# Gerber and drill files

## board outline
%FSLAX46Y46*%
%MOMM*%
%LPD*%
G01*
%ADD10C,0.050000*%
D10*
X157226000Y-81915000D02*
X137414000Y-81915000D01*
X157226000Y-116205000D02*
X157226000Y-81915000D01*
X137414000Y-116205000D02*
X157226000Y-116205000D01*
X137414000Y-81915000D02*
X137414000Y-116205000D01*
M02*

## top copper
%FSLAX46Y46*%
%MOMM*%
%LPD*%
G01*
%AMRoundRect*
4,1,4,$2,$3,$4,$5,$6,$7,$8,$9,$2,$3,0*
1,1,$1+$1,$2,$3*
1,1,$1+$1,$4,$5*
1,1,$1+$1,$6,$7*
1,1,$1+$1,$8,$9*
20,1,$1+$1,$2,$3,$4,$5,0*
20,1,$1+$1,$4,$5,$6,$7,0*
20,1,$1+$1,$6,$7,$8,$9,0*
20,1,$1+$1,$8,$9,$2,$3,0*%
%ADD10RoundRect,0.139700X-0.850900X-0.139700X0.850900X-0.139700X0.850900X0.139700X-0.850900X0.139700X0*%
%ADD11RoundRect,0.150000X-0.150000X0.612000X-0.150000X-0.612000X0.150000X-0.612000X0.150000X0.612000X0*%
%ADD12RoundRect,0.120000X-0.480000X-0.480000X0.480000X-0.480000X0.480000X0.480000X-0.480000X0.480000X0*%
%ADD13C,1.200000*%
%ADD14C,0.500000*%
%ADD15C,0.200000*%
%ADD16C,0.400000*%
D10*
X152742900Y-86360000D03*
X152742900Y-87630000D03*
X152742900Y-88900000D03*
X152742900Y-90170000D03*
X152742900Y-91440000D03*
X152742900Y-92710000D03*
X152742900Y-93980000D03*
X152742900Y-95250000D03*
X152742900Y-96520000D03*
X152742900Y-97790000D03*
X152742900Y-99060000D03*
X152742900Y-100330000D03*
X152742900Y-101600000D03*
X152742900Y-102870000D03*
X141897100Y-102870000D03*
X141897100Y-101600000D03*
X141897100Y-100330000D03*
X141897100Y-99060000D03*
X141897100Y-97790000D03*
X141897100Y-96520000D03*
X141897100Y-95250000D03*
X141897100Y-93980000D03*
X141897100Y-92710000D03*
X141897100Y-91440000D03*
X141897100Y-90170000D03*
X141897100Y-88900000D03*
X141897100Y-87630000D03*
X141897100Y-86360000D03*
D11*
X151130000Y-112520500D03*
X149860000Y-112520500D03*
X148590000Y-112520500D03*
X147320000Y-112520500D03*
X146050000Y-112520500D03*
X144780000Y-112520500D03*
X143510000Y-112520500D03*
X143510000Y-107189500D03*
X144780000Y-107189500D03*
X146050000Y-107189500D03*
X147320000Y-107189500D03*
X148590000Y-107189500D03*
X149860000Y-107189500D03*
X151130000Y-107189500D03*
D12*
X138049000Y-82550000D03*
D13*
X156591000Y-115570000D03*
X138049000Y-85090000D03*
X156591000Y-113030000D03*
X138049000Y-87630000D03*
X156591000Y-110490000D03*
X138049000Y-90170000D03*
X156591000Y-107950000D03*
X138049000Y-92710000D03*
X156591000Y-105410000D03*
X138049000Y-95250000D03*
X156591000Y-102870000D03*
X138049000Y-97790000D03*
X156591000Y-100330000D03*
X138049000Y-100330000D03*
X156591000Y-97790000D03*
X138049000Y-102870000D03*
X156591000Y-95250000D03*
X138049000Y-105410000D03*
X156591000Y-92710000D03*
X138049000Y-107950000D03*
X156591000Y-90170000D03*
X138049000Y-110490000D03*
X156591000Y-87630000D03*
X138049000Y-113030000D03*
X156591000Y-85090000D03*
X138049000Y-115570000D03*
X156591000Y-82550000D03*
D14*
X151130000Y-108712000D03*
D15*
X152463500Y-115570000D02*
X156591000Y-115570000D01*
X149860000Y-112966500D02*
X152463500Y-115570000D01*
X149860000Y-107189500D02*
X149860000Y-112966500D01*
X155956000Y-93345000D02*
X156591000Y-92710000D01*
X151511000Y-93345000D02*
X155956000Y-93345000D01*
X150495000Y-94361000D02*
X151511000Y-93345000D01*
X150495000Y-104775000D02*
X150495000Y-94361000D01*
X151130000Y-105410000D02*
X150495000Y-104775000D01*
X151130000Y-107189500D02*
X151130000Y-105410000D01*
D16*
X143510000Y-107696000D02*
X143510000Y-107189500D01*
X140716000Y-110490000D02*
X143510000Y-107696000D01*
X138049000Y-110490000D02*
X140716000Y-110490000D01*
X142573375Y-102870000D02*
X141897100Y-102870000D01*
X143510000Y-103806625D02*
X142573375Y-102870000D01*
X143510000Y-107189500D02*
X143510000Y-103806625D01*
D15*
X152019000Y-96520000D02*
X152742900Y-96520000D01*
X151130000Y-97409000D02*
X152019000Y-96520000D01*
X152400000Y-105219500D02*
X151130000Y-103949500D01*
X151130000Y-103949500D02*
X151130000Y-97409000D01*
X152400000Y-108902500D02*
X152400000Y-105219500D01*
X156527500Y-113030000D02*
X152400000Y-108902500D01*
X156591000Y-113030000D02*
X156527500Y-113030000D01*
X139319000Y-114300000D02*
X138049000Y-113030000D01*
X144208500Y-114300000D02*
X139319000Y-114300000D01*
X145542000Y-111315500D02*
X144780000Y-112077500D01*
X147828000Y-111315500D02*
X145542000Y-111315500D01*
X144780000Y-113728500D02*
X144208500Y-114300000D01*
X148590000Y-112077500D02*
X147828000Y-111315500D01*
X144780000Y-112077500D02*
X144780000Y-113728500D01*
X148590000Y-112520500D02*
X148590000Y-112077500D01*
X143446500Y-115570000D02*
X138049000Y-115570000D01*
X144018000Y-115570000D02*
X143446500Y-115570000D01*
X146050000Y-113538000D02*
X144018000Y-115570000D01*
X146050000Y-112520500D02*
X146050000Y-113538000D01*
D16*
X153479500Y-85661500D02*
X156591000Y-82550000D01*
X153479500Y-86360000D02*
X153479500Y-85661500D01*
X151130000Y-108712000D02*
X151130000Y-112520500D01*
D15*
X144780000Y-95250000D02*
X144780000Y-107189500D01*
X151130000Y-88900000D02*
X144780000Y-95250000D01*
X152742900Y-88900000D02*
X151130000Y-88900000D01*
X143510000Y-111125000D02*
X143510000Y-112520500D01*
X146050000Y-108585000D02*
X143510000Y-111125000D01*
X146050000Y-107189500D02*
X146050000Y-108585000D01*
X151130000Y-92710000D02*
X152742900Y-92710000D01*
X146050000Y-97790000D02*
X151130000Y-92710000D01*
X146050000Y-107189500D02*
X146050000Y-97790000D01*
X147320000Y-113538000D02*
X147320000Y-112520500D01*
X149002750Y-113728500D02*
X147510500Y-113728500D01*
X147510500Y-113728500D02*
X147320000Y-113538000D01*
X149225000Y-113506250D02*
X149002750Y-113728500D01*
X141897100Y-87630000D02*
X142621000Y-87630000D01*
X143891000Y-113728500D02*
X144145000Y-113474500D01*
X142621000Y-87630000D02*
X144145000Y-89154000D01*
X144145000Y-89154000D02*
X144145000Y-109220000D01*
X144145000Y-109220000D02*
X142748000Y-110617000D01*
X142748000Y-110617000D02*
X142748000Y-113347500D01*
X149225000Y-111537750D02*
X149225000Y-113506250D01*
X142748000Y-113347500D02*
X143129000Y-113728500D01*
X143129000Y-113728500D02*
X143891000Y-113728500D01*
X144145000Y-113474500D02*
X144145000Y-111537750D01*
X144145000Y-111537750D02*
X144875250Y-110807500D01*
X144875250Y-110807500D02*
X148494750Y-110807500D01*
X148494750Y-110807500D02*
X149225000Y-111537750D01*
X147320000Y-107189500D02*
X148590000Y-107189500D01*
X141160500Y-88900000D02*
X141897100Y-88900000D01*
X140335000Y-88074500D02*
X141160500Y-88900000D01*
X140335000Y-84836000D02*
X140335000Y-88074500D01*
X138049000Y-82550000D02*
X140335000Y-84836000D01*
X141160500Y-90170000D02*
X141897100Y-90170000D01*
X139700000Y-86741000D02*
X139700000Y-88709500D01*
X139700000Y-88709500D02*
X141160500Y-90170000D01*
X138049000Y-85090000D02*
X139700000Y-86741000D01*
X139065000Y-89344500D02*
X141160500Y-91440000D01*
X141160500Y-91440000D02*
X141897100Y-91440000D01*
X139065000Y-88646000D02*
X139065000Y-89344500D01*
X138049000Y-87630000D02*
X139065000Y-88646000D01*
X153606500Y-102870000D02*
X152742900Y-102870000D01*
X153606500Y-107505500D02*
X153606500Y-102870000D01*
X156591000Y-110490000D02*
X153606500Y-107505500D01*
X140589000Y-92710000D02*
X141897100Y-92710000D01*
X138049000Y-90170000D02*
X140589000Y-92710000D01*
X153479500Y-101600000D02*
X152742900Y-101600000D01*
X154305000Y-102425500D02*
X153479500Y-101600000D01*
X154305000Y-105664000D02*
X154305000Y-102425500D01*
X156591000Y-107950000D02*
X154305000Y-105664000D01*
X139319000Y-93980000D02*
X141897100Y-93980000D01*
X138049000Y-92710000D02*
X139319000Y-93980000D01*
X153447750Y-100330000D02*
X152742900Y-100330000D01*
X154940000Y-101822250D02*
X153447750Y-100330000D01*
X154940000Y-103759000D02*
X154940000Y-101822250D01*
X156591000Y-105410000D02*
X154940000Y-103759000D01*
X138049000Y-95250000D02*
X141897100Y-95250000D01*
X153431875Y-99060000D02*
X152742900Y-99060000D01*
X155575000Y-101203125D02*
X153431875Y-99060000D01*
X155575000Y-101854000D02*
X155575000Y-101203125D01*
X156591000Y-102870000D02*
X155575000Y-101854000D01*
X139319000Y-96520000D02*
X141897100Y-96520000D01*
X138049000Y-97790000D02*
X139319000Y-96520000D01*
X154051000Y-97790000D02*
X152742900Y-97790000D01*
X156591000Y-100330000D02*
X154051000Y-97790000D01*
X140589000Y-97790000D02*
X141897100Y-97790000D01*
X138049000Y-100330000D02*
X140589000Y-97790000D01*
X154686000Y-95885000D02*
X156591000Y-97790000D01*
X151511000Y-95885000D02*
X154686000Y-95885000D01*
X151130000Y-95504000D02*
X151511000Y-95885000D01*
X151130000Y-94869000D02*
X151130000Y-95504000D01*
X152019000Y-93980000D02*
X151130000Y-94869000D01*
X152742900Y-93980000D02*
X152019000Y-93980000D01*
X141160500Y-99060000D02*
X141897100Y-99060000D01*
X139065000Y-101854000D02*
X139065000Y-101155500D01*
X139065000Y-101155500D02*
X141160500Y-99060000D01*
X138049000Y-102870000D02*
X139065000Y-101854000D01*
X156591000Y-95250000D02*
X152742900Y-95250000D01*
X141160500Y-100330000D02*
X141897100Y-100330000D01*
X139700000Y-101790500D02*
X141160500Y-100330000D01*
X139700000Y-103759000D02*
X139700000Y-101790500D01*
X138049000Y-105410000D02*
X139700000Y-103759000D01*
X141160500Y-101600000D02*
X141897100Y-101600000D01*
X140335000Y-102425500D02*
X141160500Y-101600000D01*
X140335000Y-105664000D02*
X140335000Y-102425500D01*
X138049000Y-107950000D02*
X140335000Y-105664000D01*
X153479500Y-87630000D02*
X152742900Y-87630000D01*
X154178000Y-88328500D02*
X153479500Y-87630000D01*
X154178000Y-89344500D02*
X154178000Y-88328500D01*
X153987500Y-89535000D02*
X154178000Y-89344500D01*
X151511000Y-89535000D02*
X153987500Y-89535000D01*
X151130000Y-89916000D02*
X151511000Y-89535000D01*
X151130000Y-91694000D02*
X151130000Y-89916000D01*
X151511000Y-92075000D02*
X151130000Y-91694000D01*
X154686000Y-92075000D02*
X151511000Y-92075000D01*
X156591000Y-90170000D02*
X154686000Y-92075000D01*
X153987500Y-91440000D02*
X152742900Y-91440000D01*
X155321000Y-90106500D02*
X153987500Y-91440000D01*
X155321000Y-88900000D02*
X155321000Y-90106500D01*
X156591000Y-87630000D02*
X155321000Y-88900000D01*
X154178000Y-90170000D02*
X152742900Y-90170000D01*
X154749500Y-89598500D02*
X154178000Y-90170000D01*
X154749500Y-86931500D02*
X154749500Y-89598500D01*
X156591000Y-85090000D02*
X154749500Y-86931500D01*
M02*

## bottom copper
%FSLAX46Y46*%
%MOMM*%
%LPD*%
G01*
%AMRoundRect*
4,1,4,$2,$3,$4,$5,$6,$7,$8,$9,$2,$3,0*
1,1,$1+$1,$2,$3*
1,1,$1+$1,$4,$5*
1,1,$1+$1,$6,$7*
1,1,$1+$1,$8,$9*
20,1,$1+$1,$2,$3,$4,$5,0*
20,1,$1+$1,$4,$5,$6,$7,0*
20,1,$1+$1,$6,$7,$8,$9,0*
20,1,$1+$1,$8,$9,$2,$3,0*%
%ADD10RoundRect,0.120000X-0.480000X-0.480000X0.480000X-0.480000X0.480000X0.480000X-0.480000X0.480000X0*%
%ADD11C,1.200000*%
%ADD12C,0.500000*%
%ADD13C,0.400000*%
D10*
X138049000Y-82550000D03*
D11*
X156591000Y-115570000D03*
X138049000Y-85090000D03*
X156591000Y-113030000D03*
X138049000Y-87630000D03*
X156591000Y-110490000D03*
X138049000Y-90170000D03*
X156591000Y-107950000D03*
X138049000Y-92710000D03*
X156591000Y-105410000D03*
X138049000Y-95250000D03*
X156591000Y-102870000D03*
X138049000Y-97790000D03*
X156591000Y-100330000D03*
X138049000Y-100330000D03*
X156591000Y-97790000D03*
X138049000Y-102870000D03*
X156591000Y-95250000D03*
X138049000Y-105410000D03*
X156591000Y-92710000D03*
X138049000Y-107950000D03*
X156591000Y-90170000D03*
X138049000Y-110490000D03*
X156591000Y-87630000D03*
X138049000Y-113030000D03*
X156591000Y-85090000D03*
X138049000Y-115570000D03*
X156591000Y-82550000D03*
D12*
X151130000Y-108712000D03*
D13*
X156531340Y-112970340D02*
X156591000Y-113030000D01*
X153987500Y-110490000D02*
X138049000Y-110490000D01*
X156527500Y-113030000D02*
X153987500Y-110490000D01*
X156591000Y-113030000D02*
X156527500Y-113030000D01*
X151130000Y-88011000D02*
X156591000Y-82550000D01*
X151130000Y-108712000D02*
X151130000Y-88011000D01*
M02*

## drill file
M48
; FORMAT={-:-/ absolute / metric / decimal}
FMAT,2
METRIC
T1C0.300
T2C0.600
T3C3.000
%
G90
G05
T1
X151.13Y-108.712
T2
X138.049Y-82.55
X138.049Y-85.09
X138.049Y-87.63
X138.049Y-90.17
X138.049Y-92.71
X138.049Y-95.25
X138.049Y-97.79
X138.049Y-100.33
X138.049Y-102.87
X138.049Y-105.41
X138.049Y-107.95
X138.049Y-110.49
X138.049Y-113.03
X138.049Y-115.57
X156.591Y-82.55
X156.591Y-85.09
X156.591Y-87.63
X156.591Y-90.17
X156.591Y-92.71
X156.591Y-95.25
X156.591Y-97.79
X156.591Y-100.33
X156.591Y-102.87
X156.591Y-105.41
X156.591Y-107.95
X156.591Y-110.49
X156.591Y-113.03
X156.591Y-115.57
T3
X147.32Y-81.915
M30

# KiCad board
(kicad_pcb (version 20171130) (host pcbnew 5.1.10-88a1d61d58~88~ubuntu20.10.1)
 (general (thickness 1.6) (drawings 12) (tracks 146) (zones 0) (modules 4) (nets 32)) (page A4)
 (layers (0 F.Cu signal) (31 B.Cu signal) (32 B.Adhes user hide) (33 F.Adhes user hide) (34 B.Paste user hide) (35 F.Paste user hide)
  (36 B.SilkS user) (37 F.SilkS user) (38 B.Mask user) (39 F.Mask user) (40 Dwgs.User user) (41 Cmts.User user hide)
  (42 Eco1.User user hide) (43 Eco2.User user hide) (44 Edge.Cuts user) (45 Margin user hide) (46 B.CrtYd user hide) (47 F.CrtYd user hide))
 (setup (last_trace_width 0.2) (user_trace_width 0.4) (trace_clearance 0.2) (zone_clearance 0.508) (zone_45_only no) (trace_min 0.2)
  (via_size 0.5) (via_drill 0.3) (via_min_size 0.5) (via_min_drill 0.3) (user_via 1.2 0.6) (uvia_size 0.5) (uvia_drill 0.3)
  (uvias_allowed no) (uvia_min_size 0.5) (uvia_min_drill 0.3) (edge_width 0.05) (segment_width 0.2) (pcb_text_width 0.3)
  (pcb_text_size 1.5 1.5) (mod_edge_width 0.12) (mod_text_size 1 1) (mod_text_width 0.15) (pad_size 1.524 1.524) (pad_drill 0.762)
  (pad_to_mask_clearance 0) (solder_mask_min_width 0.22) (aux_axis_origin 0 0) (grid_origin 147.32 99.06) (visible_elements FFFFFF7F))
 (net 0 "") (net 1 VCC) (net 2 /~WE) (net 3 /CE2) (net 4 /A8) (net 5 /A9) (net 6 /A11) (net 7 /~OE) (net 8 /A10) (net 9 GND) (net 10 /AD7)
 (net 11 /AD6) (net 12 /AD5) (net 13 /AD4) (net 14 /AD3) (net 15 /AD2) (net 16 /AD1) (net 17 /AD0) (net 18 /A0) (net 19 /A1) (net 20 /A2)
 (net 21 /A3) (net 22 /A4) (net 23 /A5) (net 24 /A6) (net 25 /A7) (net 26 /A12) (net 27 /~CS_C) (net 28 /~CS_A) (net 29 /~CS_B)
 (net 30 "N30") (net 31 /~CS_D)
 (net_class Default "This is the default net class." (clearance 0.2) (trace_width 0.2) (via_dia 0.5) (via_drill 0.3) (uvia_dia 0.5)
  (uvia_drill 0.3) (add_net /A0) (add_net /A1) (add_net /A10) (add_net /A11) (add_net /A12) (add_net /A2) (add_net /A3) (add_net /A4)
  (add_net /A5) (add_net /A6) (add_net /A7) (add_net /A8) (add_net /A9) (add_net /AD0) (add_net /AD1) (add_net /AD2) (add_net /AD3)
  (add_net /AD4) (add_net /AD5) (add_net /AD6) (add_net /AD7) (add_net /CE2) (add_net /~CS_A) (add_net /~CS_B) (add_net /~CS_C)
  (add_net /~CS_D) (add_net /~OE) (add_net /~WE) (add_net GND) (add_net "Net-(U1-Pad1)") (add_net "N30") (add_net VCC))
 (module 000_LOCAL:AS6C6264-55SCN (layer F.Cu) (at 147.32 94.615)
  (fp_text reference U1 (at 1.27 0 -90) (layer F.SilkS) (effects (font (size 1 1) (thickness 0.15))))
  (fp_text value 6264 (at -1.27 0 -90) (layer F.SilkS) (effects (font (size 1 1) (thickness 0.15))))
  (pad 28 smd roundrect (at 5.4229 -8.255) (size 1.9812 0.5588) (layers F.Cu F.Paste F.Mask) (roundrect_rratio 0.25) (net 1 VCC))
  (pad 27 smd roundrect (at 5.4229 -6.985) (size 1.9812 0.5588) (layers F.Cu F.Paste F.Mask) (roundrect_rratio 0.25) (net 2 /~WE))
  (pad 26 smd roundrect (at 5.4229 -5.715) (size 1.9812 0.5588) (layers F.Cu F.Paste F.Mask) (roundrect_rratio 0.25) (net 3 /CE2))
  (pad 25 smd roundrect (at 5.4229 -4.445) (size 1.9812 0.5588) (layers F.Cu F.Paste F.Mask) (roundrect_rratio 0.25) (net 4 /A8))
  (pad 24 smd roundrect (at 5.4229 -3.175) (size 1.9812 0.5588) (layers F.Cu F.Paste F.Mask) (roundrect_rratio 0.25) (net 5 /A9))
  (pad 23 smd roundrect (at 5.4229 -1.905) (size 1.9812 0.5588) (layers F.Cu F.Paste F.Mask) (roundrect_rratio 0.25) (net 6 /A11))
  (pad 22 smd roundrect (at 5.4229 -0.635) (size 1.9812 0.5588) (layers F.Cu F.Paste F.Mask) (roundrect_rratio 0.25) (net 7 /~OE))
  (pad 21 smd roundrect (at 5.4229 0.635) (size 1.9812 0.5588) (layers F.Cu F.Paste F.Mask) (roundrect_rratio 0.25) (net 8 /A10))
  (pad 20 smd roundrect (at 5.4229 1.905) (size 1.9812 0.5588) (layers F.Cu F.Paste F.Mask) (roundrect_rratio 0.25) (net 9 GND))
  (pad 19 smd roundrect (at 5.4229 3.175) (size 1.9812 0.5588) (layers F.Cu F.Paste F.Mask) (roundrect_rratio 0.25) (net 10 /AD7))
  (pad 18 smd roundrect (at 5.4229 4.445) (size 1.9812 0.5588) (layers F.Cu F.Paste F.Mask) (roundrect_rratio 0.25) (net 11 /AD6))
  (pad 17 smd roundrect (at 5.4229 5.715) (size 1.9812 0.5588) (layers F.Cu F.Paste F.Mask) (roundrect_rratio 0.25) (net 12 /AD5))
  (pad 16 smd roundrect (at 5.4229 6.985) (size 1.9812 0.5588) (layers F.Cu F.Paste F.Mask) (roundrect_rratio 0.25) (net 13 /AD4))
  (pad 15 smd roundrect (at 5.4229 8.255) (size 1.9812 0.5588) (layers F.Cu F.Paste F.Mask) (roundrect_rratio 0.25) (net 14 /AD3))
  (pad 14 smd roundrect (at -5.4229 8.255) (size 1.9812 0.5588) (layers F.Cu F.Paste F.Mask) (roundrect_rratio 0.25) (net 9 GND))
  (pad 13 smd roundrect (at -5.4229 6.985) (size 1.9812 0.5588) (layers F.Cu F.Paste F.Mask) (roundrect_rratio 0.25) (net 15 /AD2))
  (pad 12 smd roundrect (at -5.4229 5.715) (size 1.9812 0.5588) (layers F.Cu F.Paste F.Mask) (roundrect_rratio 0.25) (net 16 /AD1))
  (pad 11 smd roundrect (at -5.4229 4.445) (size 1.9812 0.5588) (layers F.Cu F.Paste F.Mask) (roundrect_rratio 0.25) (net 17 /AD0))
  (pad 10 smd roundrect (at -5.4229 3.175) (size 1.9812 0.5588) (layers F.Cu F.Paste F.Mask) (roundrect_rratio 0.25) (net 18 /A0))
  (pad 9 smd roundrect (at -5.4229 1.905) (size 1.9812 0.5588) (layers F.Cu F.Paste F.Mask) (roundrect_rratio 0.25) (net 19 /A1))
  (pad 8 smd roundrect (at -5.4229 0.635) (size 1.9812 0.5588) (layers F.Cu F.Paste F.Mask) (roundrect_rratio 0.25) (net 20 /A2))
  (pad 7 smd roundrect (at -5.4229 -0.635) (size 1.9812 0.5588) (layers F.Cu F.Paste F.Mask) (roundrect_rratio 0.25) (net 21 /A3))
  (pad 6 smd roundrect (at -5.4229 -1.905) (size 1.9812 0.5588) (layers F.Cu F.Paste F.Mask) (roundrect_rratio 0.25) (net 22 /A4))
  (pad 5 smd roundrect (at -5.4229 -3.175) (size 1.9812 0.5588) (layers F.Cu F.Paste F.Mask) (roundrect_rratio 0.25) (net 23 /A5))
  (pad 4 smd roundrect (at -5.4229 -4.445) (size 1.9812 0.5588) (layers F.Cu F.Paste F.Mask) (roundrect_rratio 0.25) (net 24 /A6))
  (pad 3 smd roundrect (at -5.4229 -5.715) (size 1.9812 0.5588) (layers F.Cu F.Paste F.Mask) (roundrect_rratio 0.25) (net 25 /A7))
  (pad 2 smd roundrect (at -5.4229 -6.985) (size 1.9812 0.5588) (layers F.Cu F.Paste F.Mask) (roundrect_rratio 0.25) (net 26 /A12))
  (pad 1 smd roundrect (at -5.4229 -8.255) (size 1.9812 0.5588) (layers F.Cu F.Paste F.Mask) (roundrect_rratio 0.25)))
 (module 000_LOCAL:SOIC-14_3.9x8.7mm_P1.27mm (layer F.Cu) (at 147.32 109.855 270) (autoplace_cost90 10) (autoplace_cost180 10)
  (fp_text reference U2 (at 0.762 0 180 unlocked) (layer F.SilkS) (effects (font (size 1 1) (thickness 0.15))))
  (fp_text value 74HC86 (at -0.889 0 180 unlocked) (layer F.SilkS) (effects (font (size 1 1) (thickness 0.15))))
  (pad 14 smd roundrect (at 2.6655 -3.81 270) (size 1.524 0.6) (layers F.Cu F.Paste F.Mask) (roundrect_rratio 0.25) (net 1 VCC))
  (pad 13 smd roundrect (at 2.6655 -2.54 270) (size 1.524 0.6) (layers F.Cu F.Paste F.Mask) (roundrect_rratio 0.25) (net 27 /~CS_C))
  (pad 12 smd roundrect (at 2.6655 -1.27 270) (size 1.524 0.6) (layers F.Cu F.Paste F.Mask) (roundrect_rratio 0.25) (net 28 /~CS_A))
  (pad 11 smd roundrect (at 2.6655 0 270) (size 1.524 0.6) (layers F.Cu F.Paste F.Mask) (roundrect_rratio 0.25) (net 26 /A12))
  (pad 10 smd roundrect (at 2.6655 1.27 270) (size 1.524 0.6) (layers F.Cu F.Paste F.Mask) (roundrect_rratio 0.25) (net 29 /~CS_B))
  (pad 9 smd roundrect (at 2.6655 2.54 270) (size 1.524 0.6) (layers F.Cu F.Paste F.Mask) (roundrect_rratio 0.25) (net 28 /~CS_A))
  (pad 8 smd roundrect (at 2.6655 3.81 270) (size 1.524 0.6) (layers F.Cu F.Paste F.Mask) (roundrect_rratio 0.25) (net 6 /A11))
  (pad 7 smd roundrect (at -2.6655 3.81 270) (size 1.524 0.6) (layers F.Cu F.Paste F.Mask) (roundrect_rratio 0.25) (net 9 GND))
  (pad 6 smd roundrect (at -2.6655 2.54 270) (size 1.524 0.6) (layers F.Cu F.Paste F.Mask) (roundrect_rratio 0.25) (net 3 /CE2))
  (pad 5 smd roundrect (at -2.6655 1.27 270) (size 1.524 0.6) (layers F.Cu F.Paste F.Mask) (roundrect_rratio 0.25) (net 6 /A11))
  (pad 4 smd roundrect (at -2.6655 0 270) (size 1.524 0.6) (layers F.Cu F.Paste F.Mask) (roundrect_rratio 0.25) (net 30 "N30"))
  (pad 3 smd roundrect (at -2.6655 -1.27 270) (size 1.524 0.6) (layers F.Cu F.Paste F.Mask) (roundrect_rratio 0.25) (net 30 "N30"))
  (pad 2 smd roundrect (at -2.6655 -2.54 270) (size 1.524 0.6) (layers F.Cu F.Paste F.Mask) (roundrect_rratio 0.25) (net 27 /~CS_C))
  (pad 1 smd roundrect (at -2.6655 -3.81 270) (size 1.524 0.6) (layers F.Cu F.Paste F.Mask) (roundrect_rratio 0.25) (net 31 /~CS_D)))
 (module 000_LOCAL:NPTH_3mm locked (layer F.Cu) (at 147.32 81.915)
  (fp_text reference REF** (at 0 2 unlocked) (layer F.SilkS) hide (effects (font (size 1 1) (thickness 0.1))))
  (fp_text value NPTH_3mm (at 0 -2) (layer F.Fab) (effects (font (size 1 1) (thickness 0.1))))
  (pad "" np_thru_hole circle (at 0 0) (size 3 3) (drill 3) (layers *.Cu *.Mask)))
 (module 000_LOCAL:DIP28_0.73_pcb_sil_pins (layer F.Cu) (at 147.32 99.06)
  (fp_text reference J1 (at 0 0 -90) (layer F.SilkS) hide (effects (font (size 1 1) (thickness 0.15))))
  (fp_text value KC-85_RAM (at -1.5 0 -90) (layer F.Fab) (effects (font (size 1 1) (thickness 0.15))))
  (pad 1 thru_hole roundrect (at -9.271 -16.51) (size 1.2 1.2) (drill 0.6) (layers *.Cu *.Mask) (roundrect_rratio 0.1) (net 25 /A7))
  (pad 15 thru_hole circle (at 9.271 16.51) (size 1.2 1.2) (drill 0.6) (layers *.Cu *.Mask) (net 27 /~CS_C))
  (pad 2 thru_hole circle (at -9.271 -13.97) (size 1.2 1.2) (drill 0.6) (layers *.Cu *.Mask) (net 24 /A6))
  (pad 16 thru_hole circle (at 9.271 13.97) (size 1.2 1.2) (drill 0.6) (layers *.Cu *.Mask) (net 9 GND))
  (pad 3 thru_hole circle (at -9.271 -11.43) (size 1.2 1.2) (drill 0.6) (layers *.Cu *.Mask) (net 23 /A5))
  (pad 17 thru_hole circle (at 9.271 11.43) (size 1.2 1.2) (drill 0.6) (layers *.Cu *.Mask) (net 14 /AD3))
  (pad 4 thru_hole circle (at -9.271 -8.89) (size 1.2 1.2) (drill 0.6) (layers *.Cu *.Mask) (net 22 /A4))
  (pad 18 thru_hole circle (at 9.271 8.89) (size 1.2 1.2) (drill 0.6) (layers *.Cu *.Mask) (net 13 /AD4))
  (pad 5 thru_hole circle (at -9.271 -6.35) (size 1.2 1.2) (drill 0.6) (layers *.Cu *.Mask) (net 21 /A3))
  (pad 19 thru_hole circle (at 9.271 6.35) (size 1.2 1.2) (drill 0.6) (layers *.Cu *.Mask) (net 12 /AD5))
  (pad 6 thru_hole circle (at -9.271 -3.81) (size 1.2 1.2) (drill 0.6) (layers *.Cu *.Mask) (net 20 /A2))
  (pad 20 thru_hole circle (at 9.271 3.81) (size 1.2 1.2) (drill 0.6) (layers *.Cu *.Mask) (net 11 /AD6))
  (pad 7 thru_hole circle (at -9.271 -1.27) (size 1.2 1.2) (drill 0.6) (layers *.Cu *.Mask) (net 19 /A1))
  (pad 21 thru_hole circle (at 9.271 1.27) (size 1.2 1.2) (drill 0.6) (layers *.Cu *.Mask) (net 10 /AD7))
  (pad 8 thru_hole circle (at -9.271 1.27) (size 1.2 1.2) (drill 0.6) (layers *.Cu *.Mask) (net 18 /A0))
  (pad 22 thru_hole circle (at 9.271 -1.27) (size 1.2 1.2) (drill 0.6) (layers *.Cu *.Mask) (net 7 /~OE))
  (pad 9 thru_hole circle (at -9.271 3.81) (size 1.2 1.2) (drill 0.6) (layers *.Cu *.Mask) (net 17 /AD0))
  (pad 23 thru_hole circle (at 9.271 -3.81) (size 1.2 1.2) (drill 0.6) (layers *.Cu *.Mask) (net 8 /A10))
  (pad 10 thru_hole circle (at -9.271 6.35) (size 1.2 1.2) (drill 0.6) (layers *.Cu *.Mask) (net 16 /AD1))
  (pad 24 thru_hole circle (at 9.271 -6.35) (size 1.2 1.2) (drill 0.6) (layers *.Cu *.Mask) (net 31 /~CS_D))
  (pad 11 thru_hole circle (at -9.271 8.89) (size 1.2 1.2) (drill 0.6) (layers *.Cu *.Mask) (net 15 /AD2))
  (pad 25 thru_hole circle (at 9.271 -8.89) (size 1.2 1.2) (drill 0.6) (layers *.Cu *.Mask) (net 2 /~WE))
  (pad 12 thru_hole circle (at -9.271 11.43) (size 1.2 1.2) (drill 0.6) (layers *.Cu *.Mask) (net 9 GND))
  (pad 26 thru_hole circle (at 9.271 -11.43) (size 1.2 1.2) (drill 0.6) (layers *.Cu *.Mask) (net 5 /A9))
  (pad 13 thru_hole circle (at -9.271 13.97) (size 1.2 1.2) (drill 0.6) (layers *.Cu *.Mask) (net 28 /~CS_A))
  (pad 27 thru_hole circle (at 9.271 -13.97) (size 1.2 1.2) (drill 0.6) (layers *.Cu *.Mask) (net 4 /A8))
  (pad 14 thru_hole circle (at -9.271 16.51) (size 1.2 1.2) (drill 0.6) (layers *.Cu *.Mask) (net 29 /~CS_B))
  (pad 28 thru_hole circle (at 9.271 -16.51) (size 1.2 1.2) (drill 0.6) (layers *.Cu *.Mask) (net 1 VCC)))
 (gr_line (start 157.226 81.915) (end 137.414 81.915) (layer Edge.Cuts) (width 0.05))
 (gr_line (start 157.226 116.205) (end 157.226 81.915) (layer Edge.Cuts) (width 0.05))
 (gr_line (start 137.414 116.205) (end 157.226 116.205) (layer Edge.Cuts) (width 0.05))
 (gr_line (start 137.414 81.915) (end 137.414 116.205) (layer Edge.Cuts) (width 0.05))
 (segment (start 152.4635 115.57) (end 156.591 115.57) (width 0.2) (layer F.Cu) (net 27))
 (segment (start 149.86 112.9665) (end 152.4635 115.57) (width 0.2) (layer F.Cu) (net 27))
 (segment (start 149.86 107.1895) (end 149.86 112.9665) (width 0.2) (layer F.Cu) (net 27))
 (segment (start 155.956 93.345) (end 156.591 92.71) (width 0.2) (layer F.Cu) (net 31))
 (segment (start 151.511 93.345) (end 155.956 93.345) (width 0.2) (layer F.Cu) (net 31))
 (segment (start 150.495 94.361) (end 151.511 93.345) (width 0.2) (layer F.Cu) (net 31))
 (segment (start 150.495 104.775) (end 150.495 94.361) (width 0.2) (layer F.Cu) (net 31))
 (segment (start 151.13 105.41) (end 150.495 104.775) (width 0.2) (layer F.Cu) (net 31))
 (segment (start 151.13 107.1895) (end 151.13 105.41) (width 0.2) (layer F.Cu) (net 31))
 (segment (start 156.53134 112.97034) (end 156.591 113.03) (width 0.4) (layer B.Cu) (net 9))
 (segment (start 143.51 107.696) (end 143.51 107.1895) (width 0.4) (layer F.Cu) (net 9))
 (segment (start 140.716 110.49) (end 143.51 107.696) (width 0.4) (layer F.Cu) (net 9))
 (segment (start 138.049 110.49) (end 140.716 110.49) (width 0.4) (layer F.Cu) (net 9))
 (segment (start 142.573375 102.87) (end 141.8971 102.87) (width 0.4) (layer F.Cu) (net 9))
 (segment (start 143.51 103.806625) (end 142.573375 102.87) (width 0.4) (layer F.Cu) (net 9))
 (segment (start 143.51 107.1895) (end 143.51 103.806625) (width 0.4) (layer F.Cu) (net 9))
 (segment (start 152.019 96.52) (end 152.7429 96.52) (width 0.2) (layer F.Cu) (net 9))
 (segment (start 151.13 97.409) (end 152.019 96.52) (width 0.2) (layer F.Cu) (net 9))
 (segment (start 152.4 105.2195) (end 151.13 103.9495) (width 0.2) (layer F.Cu) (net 9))
 (segment (start 151.13 103.9495) (end 151.13 97.409) (width 0.2) (layer F.Cu) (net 9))
 (segment (start 152.4 108.9025) (end 152.4 105.2195) (width 0.2) (layer F.Cu) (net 9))
 (segment (start 156.5275 113.03) (end 152.4 108.9025) (width 0.2) (layer F.Cu) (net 9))
 (segment (start 156.591 113.03) (end 156.5275 113.03) (width 0.2) (layer F.Cu) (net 9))
 (segment (start 153.9875 110.49) (end 138.049 110.49) (width 0.4) (layer B.Cu) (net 9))
 (segment (start 156.5275 113.03) (end 153.9875 110.49) (width 0.4) (layer B.Cu) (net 9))
 (segment (start 156.591 113.03) (end 156.5275 113.03) (width 0.4) (layer B.Cu) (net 9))
 (segment (start 139.319 114.3) (end 138.049 113.03) (width 0.2) (layer F.Cu) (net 28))
 (segment (start 144.2085 114.3) (end 139.319 114.3) (width 0.2) (layer F.Cu) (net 28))
 (segment (start 145.542 111.3155) (end 144.78 112.0775) (width 0.2) (layer F.Cu) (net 28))
 (segment (start 147.828 111.3155) (end 145.542 111.3155) (width 0.2) (layer F.Cu) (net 28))
 (segment (start 144.78 113.7285) (end 144.2085 114.3) (width 0.2) (layer F.Cu) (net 28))
 (segment (start 148.59 112.0775) (end 147.828 111.3155) (width 0.2) (layer F.Cu) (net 28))
 (segment (start 144.78 112.0775) (end 144.78 113.7285) (width 0.2) (layer F.Cu) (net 28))
 (segment (start 148.59 112.5205) (end 148.59 112.0775) (width 0.2) (layer F.Cu) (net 28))
 (segment (start 143.4465 115.57) (end 138.049 115.57) (width 0.2) (layer F.Cu) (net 29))
 (segment (start 144.018 115.57) (end 143.4465 115.57) (width 0.2) (layer F.Cu) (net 29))
 (segment (start 146.05 113.538) (end 144.018 115.57) (width 0.2) (layer F.Cu) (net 29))
 (segment (start 146.05 112.5205) (end 146.05 113.538) (width 0.2) (layer F.Cu) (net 29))
 (segment (start 153.4795 85.6615) (end 156.591 82.55) (width 0.4) (layer F.Cu) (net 1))
 (segment (start 153.4795 86.36) (end 153.4795 85.6615) (width 0.4) (layer F.Cu) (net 1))
 (segment (start 151.13 88.011) (end 156.591 82.55) (width 0.4) (layer B.Cu) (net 1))
 (segment (start 151.13 108.712) (end 151.13 88.011) (width 0.4) (layer B.Cu) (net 1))
 (segment (start 151.13 108.712) (end 151.13 112.5205) (width 0.4) (layer F.Cu) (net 1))
 (via (at 151.13 108.712) (size 0.5) (drill 0.3) (layers F.Cu B.Cu) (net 1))
 (segment (start 144.78 95.25) (end 144.78 107.1895) (width 0.2) (layer F.Cu) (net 3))
 (segment (start 151.13 88.9) (end 144.78 95.25) (width 0.2) (layer F.Cu) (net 3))
 (segment (start 152.7429 88.9) (end 151.13 88.9) (width 0.2) (layer F.Cu) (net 3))
 (segment (start 143.51 111.125) (end 143.51 112.5205) (width 0.2) (layer F.Cu) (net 6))
 (segment (start 146.05 108.585) (end 143.51 111.125) (width 0.2) (layer F.Cu) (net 6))
 (segment (start 146.05 107.1895) (end 146.05 108.585) (width 0.2) (layer F.Cu) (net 6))
 (segment (start 151.13 92.71) (end 152.7429 92.71) (width 0.2) (layer F.Cu) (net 6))
 (segment (start 146.05 97.79) (end 151.13 92.71) (width 0.2) (layer F.Cu) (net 6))
 (segment (start 146.05 107.1895) (end 146.05 97.79) (width 0.2) (layer F.Cu) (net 6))
 (segment (start 147.32 113.538) (end 147.32 112.5205) (width 0.2) (layer F.Cu) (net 26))
 (segment (start 149.00275 113.7285) (end 147.5105 113.7285) (width 0.2) (layer F.Cu) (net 26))
 (segment (start 147.5105 113.7285) (end 147.32 113.538) (width 0.2) (layer F.Cu) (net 26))
 (segment (start 149.225 113.50625) (end 149.00275 113.7285) (width 0.2) (layer F.Cu) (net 26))
 (segment (start 141.8971 87.63) (end 142.621 87.63) (width 0.2) (layer F.Cu) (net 26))
 (segment (start 143.891 113.7285) (end 144.145 113.4745) (width 0.2) (layer F.Cu) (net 26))
 (segment (start 142.621 87.63) (end 144.145 89.154) (width 0.2) (layer F.Cu) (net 26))
 (segment (start 144.145 89.154) (end 144.145 109.22) (width 0.2) (layer F.Cu) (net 26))
 (segment (start 144.145 109.22) (end 142.748 110.617) (width 0.2) (layer F.Cu) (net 26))
 (segment (start 142.748 110.617) (end 142.748 113.3475) (width 0.2) (layer F.Cu) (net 26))
 (segment (start 149.225 111.53775) (end 149.225 113.50625) (width 0.2) (layer F.Cu) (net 26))
 (segment (start 142.748 113.3475) (end 143.129 113.7285) (width 0.2) (layer F.Cu) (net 26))
 (segment (start 143.129 113.7285) (end 143.891 113.7285) (width 0.2) (layer F.Cu) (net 26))
 (segment (start 144.145 113.4745) (end 144.145 111.53775) (width 0.2) (layer F.Cu) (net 26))
 (segment (start 144.145 111.53775) (end 144.87525 110.8075) (width 0.2) (layer F.Cu) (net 26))
 (segment (start 144.87525 110.8075) (end 148.49475 110.8075) (width 0.2) (layer F.Cu) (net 26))
 (segment (start 148.49475 110.8075) (end 149.225 111.53775) (width 0.2) (layer F.Cu) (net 26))
 (segment (start 147.32 107.1895) (end 148.59 107.1895) (width 0.2) (layer F.Cu) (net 30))
 (segment (start 141.1605 88.9) (end 141.8971 88.9) (width 0.2) (layer F.Cu) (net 25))
 (segment (start 140.335 88.0745) (end 141.1605 88.9) (width 0.2) (layer F.Cu) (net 25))
 (segment (start 140.335 84.836) (end 140.335 88.0745) (width 0.2) (layer F.Cu) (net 25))
 (segment (start 138.049 82.55) (end 140.335 84.836) (width 0.2) (layer F.Cu) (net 25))
 (segment (start 141.1605 90.17) (end 141.8971 90.17) (width 0.2) (layer F.Cu) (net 24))
 (segment (start 139.7 86.741) (end 139.7 88.7095) (width 0.2) (layer F.Cu) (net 24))
 (segment (start 139.7 88.7095) (end 141.1605 90.17) (width 0.2) (layer F.Cu) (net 24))
 (segment (start 138.049 85.09) (end 139.7 86.741) (width 0.2) (layer F.Cu) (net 24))
 (segment (start 139.065 89.3445) (end 141.1605 91.44) (width 0.2) (layer F.Cu) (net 23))
 (segment (start 141.1605 91.44) (end 141.8971 91.44) (width 0.2) (layer F.Cu) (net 23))
 (segment (start 139.065 88.646) (end 139.065 89.3445) (width 0.2) (layer F.Cu) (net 23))
 (segment (start 138.049 87.63) (end 139.065 88.646) (width 0.2) (layer F.Cu) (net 23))
 (segment (start 153.6065 102.87) (end 152.7429 102.87) (width 0.2) (layer F.Cu) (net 14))
 (segment (start 153.6065 107.5055) (end 153.6065 102.87) (width 0.2) (layer F.Cu) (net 14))
 (segment (start 156.591 110.49) (end 153.6065 107.5055) (width 0.2) (layer F.Cu) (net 14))
 (segment (start 140.589 92.71) (end 141.8971 92.71) (width 0.2) (layer F.Cu) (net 22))
 (segment (start 138.049 90.17) (end 140.589 92.71) (width 0.2) (layer F.Cu) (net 22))
 (segment (start 153.4795 101.6) (end 152.7429 101.6) (width 0.2) (layer F.Cu) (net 13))
 (segment (start 154.305 102.4255) (end 153.4795 101.6) (width 0.2) (layer F.Cu) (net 13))
 (segment (start 154.305 105.664) (end 154.305 102.4255) (width 0.2) (layer F.Cu) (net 13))
 (segment (start 156.591 107.95) (end 154.305 105.664) (width 0.2) (layer F.Cu) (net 13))
 (segment (start 139.319 93.98) (end 141.8971 93.98) (width 0.2) (layer F.Cu) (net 21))
 (segment (start 138.049 92.71) (end 139.319 93.98) (width 0.2) (layer F.Cu) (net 21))
 (segment (start 153.44775 100.33) (end 152.7429 100.33) (width 0.2) (layer F.Cu) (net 12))
 (segment (start 154.94 101.82225) (end 153.44775 100.33) (width 0.2) (layer F.Cu) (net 12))
 (segment (start 154.94 103.759) (end 154.94 101.82225) (width 0.2) (layer F.Cu) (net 12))
 (segment (start 156.591 105.41) (end 154.94 103.759) (width 0.2) (layer F.Cu) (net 12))
 (segment (start 138.049 95.25) (end 141.8971 95.25) (width 0.2) (layer F.Cu) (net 20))
 (segment (start 153.431875 99.06) (end 152.7429 99.06) (width 0.2) (layer F.Cu) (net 11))
 (segment (start 155.575 101.203125) (end 153.431875 99.06) (width 0.2) (layer F.Cu) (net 11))
 (segment (start 155.575 101.854) (end 155.575 101.203125) (width 0.2) (layer F.Cu) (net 11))
 (segment (start 156.591 102.87) (end 155.575 101.854) (width 0.2) (layer F.Cu) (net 11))
 (segment (start 139.319 96.52) (end 141.8971 96.52) (width 0.2) (layer F.Cu) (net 19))
 (segment (start 138.049 97.79) (end 139.319 96.52) (width 0.2) (layer F.Cu) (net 19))
 (segment (start 154.051 97.79) (end 152.7429 97.79) (width 0.2) (layer F.Cu) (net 10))
 (segment (start 156.591 100.33) (end 154.051 97.79) (width 0.2) (layer F.Cu) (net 10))
 (segment (start 140.589 97.79) (end 141.8971 97.79) (width 0.2) (layer F.Cu) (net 18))
 (segment (start 138.049 100.33) (end 140.589 97.79) (width 0.2) (layer F.Cu) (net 18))
 (segment (start 154.686 95.885) (end 156.591 97.79) (width 0.2) (layer F.Cu) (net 7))
 (segment (start 151.511 95.885) (end 154.686 95.885) (width 0.2) (layer F.Cu) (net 7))
 (segment (start 151.13 95.504) (end 151.511 95.885) (width 0.2) (layer F.Cu) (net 7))
 (segment (start 151.13 94.869) (end 151.13 95.504) (width 0.2) (layer F.Cu) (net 7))
 (segment (start 152.019 93.98) (end 151.13 94.869) (width 0.2) (layer F.Cu) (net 7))
 (segment (start 152.7429 93.98) (end 152.019 93.98) (width 0.2) (layer F.Cu) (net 7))
 (segment (start 141.1605 99.06) (end 141.8971 99.06) (width 0.2) (layer F.Cu) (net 17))
 (segment (start 139.065 101.854) (end 139.065 101.1555) (width 0.2) (layer F.Cu) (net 17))
 (segment (start 139.065 101.1555) (end 141.1605 99.06) (width 0.2) (layer F.Cu) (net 17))
 (segment (start 138.049 102.87) (end 139.065 101.854) (width 0.2) (layer F.Cu) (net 17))
 (segment (start 156.591 95.25) (end 152.7429 95.25) (width 0.2) (layer F.Cu) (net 8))
 (segment (start 141.1605 100.33) (end 141.8971 100.33) (width 0.2) (layer F.Cu) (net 16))
 (segment (start 139.7 101.7905) (end 141.1605 100.33) (width 0.2) (layer F.Cu) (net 16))
 (segment (start 139.7 103.759) (end 139.7 101.7905) (width 0.2) (layer F.Cu) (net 16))
 (segment (start 138.049 105.41) (end 139.7 103.759) (width 0.2) (layer F.Cu) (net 16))
 (segment (start 141.1605 101.6) (end 141.8971 101.6) (width 0.2) (layer F.Cu) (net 15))
 (segment (start 140.335 102.4255) (end 141.1605 101.6) (width 0.2) (layer F.Cu) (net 15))
 (segment (start 140.335 105.664) (end 140.335 102.4255) (width 0.2) (layer F.Cu) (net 15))
 (segment (start 138.049 107.95) (end 140.335 105.664) (width 0.2) (layer F.Cu) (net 15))
 (segment (start 153.4795 87.63) (end 152.7429 87.63) (width 0.2) (layer F.Cu) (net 2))
 (segment (start 154.178 88.3285) (end 153.4795 87.63) (width 0.2) (layer F.Cu) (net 2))
 (segment (start 154.178 89.3445) (end 154.178 88.3285) (width 0.2) (layer F.Cu) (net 2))
 (segment (start 153.9875 89.535) (end 154.178 89.3445) (width 0.2) (layer F.Cu) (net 2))
 (segment (start 151.511 89.535) (end 153.9875 89.535) (width 0.2) (layer F.Cu) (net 2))
 (segment (start 151.13 89.916) (end 151.511 89.535) (width 0.2) (layer F.Cu) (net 2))
 (segment (start 151.13 91.694) (end 151.13 89.916) (width 0.2) (layer F.Cu) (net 2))
 (segment (start 151.511 92.075) (end 151.13 91.694) (width 0.2) (layer F.Cu) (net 2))
 (segment (start 154.686 92.075) (end 151.511 92.075) (width 0.2) (layer F.Cu) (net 2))
 (segment (start 156.591 90.17) (end 154.686 92.075) (width 0.2) (layer F.Cu) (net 2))
 (segment (start 153.9875 91.44) (end 152.7429 91.44) (width 0.2) (layer F.Cu) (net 5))
 (segment (start 155.321 90.1065) (end 153.9875 91.44) (width 0.2) (layer F.Cu) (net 5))
 (segment (start 155.321 88.9) (end 155.321 90.1065) (width 0.2) (layer F.Cu) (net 5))
 (segment (start 156.591 87.63) (end 155.321 88.9) (width 0.2) (layer F.Cu) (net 5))
 (segment (start 154.178 90.17) (end 152.7429 90.17) (width 0.2) (layer F.Cu) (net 4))
 (segment (start 154.7495 89.5985) (end 154.178 90.17) (width 0.2) (layer F.Cu) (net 4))
 (segment (start 154.7495 86.9315) (end 154.7495 89.5985) (width 0.2) (layer F.Cu) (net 4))
 (segment (start 156.591 85.09) (end 154.7495 86.9315) (width 0.2) (layer F.Cu) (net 4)))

